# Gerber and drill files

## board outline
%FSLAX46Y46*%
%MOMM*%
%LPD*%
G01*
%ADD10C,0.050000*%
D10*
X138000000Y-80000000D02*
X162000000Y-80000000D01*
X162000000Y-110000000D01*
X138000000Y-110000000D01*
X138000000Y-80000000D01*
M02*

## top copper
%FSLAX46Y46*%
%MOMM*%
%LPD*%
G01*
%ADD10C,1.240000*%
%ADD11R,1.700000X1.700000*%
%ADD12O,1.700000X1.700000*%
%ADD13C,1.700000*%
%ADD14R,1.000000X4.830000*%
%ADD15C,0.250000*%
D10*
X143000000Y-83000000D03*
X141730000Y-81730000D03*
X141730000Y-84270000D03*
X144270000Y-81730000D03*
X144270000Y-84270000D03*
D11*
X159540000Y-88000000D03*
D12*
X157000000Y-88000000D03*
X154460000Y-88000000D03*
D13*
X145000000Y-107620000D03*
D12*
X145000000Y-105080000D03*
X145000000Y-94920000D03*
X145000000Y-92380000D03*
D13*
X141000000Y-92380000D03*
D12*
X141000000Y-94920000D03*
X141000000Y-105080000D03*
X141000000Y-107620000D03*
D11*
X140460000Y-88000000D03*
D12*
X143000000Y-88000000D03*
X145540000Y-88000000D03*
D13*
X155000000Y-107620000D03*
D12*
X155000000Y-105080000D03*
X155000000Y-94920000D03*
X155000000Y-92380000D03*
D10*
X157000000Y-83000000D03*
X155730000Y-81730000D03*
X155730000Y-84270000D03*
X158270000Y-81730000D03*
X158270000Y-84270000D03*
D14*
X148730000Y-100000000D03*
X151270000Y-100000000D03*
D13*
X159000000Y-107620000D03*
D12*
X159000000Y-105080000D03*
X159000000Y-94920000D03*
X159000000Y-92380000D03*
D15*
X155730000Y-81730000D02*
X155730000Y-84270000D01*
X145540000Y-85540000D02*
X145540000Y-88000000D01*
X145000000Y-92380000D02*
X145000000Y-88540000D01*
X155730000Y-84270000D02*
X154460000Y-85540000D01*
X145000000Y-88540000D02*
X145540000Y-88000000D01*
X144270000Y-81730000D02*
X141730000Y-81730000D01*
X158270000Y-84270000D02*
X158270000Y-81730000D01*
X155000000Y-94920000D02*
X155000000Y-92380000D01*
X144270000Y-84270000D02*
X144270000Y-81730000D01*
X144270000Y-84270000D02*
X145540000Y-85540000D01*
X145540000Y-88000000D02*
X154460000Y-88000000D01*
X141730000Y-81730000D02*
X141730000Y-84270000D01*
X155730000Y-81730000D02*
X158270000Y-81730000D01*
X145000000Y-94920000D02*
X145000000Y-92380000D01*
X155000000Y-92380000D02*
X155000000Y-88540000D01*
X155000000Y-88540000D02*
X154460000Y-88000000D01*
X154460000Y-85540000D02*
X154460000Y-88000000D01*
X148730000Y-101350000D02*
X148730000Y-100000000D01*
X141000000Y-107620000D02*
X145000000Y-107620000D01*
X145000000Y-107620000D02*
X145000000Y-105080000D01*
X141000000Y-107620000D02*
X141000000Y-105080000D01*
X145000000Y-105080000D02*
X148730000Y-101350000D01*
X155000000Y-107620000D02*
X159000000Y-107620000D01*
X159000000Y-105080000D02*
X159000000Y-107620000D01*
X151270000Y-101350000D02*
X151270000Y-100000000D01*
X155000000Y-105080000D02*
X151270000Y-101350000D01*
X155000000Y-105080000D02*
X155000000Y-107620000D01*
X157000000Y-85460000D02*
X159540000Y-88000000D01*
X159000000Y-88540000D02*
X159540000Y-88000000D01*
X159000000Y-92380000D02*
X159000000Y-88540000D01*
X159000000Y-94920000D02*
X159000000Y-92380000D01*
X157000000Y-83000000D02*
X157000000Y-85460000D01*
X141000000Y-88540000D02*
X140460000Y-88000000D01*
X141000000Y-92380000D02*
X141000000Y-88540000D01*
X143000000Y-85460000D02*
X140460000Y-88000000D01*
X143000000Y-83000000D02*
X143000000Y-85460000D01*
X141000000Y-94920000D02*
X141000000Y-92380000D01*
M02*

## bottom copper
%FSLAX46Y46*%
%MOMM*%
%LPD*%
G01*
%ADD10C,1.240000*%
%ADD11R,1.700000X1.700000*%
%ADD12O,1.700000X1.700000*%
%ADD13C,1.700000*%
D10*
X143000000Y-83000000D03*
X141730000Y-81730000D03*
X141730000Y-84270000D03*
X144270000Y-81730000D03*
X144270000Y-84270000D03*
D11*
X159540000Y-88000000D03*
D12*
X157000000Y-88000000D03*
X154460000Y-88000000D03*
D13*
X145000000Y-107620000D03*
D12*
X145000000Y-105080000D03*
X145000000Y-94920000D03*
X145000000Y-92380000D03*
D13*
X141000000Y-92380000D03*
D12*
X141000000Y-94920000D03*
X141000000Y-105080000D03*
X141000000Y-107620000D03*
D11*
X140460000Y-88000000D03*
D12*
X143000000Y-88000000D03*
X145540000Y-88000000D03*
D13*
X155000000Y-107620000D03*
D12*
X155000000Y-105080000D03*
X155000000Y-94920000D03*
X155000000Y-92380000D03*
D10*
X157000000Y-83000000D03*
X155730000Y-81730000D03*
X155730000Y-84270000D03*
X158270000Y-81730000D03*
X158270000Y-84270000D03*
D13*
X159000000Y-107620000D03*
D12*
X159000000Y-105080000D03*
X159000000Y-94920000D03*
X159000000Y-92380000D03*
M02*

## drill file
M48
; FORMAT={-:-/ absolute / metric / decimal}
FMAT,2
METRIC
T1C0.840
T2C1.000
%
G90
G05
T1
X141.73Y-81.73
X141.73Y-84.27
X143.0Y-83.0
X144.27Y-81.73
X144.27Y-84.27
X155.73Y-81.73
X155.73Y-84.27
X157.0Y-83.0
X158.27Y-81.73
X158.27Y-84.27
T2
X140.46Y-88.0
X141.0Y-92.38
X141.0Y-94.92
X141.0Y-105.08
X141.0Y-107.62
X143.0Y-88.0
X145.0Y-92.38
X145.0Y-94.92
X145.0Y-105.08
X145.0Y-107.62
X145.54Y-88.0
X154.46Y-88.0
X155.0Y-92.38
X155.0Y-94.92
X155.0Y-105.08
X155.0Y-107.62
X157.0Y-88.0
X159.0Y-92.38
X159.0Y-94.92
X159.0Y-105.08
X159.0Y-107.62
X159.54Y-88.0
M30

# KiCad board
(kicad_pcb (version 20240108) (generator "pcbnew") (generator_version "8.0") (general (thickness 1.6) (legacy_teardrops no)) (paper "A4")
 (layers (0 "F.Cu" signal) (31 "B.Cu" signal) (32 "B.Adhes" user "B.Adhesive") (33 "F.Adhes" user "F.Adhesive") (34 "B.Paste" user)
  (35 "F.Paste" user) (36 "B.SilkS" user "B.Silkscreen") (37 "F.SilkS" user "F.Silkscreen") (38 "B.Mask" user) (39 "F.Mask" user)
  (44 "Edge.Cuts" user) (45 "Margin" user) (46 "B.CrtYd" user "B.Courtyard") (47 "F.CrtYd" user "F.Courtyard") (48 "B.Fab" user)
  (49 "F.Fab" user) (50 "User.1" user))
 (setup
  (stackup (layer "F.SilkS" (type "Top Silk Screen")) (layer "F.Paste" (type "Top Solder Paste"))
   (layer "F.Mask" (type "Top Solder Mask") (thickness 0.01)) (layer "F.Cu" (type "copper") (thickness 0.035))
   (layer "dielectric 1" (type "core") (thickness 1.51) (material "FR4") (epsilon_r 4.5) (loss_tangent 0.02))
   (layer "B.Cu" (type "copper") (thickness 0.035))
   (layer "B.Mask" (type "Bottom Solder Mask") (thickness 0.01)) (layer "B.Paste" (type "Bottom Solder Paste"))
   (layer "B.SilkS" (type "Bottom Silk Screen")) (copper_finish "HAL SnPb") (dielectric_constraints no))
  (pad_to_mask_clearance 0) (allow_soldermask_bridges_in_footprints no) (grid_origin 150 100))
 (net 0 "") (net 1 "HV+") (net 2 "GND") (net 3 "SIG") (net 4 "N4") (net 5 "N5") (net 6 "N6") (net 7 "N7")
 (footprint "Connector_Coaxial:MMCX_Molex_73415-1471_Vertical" (layer "F.Cu") (at 143 83)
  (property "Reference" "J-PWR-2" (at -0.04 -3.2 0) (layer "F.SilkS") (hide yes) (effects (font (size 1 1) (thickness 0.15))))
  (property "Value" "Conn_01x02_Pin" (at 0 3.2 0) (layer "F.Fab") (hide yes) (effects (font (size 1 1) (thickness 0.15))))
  (pad "1" thru_hole circle (at 0 0) (size 1.24 1.24) (drill 0.84) (layers "*.Cu" "*.Mask") (remove_unused_layers no) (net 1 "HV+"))
  (pad "2" thru_hole circle (at -1.27 -1.27) (size 1.24 1.24) (drill 0.84) (layers "*.Cu" "*.Mask") (remove_unused_layers no) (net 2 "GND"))
  (pad "2" thru_hole circle (at -1.27 1.27) (size 1.24 1.24) (drill 0.84) (layers "*.Cu" "*.Mask") (remove_unused_layers no) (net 2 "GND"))
  (pad "2" thru_hole circle (at 1.27 -1.27) (size 1.24 1.24) (drill 0.84) (layers "*.Cu" "*.Mask") (remove_unused_layers no) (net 2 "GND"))
  (pad "2" thru_hole circle (at 1.27 1.27) (size 1.24 1.24) (drill 0.84) (layers "*.Cu" "*.Mask") (remove_unused_layers no) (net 2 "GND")))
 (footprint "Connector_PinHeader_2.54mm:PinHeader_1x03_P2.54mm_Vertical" (layer "F.Cu") (at 159.54 88 -90)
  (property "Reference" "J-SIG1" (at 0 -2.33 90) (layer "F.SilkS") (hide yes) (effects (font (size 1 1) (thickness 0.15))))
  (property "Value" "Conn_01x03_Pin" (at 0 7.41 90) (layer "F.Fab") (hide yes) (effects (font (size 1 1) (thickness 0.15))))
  (pad "1" thru_hole rect (at 0 0 270) (size 1.7 1.7) (drill 1) (layers "*.Cu" "*.Mask") (remove_unused_layers no) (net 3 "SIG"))
  (pad "2" thru_hole oval (at 0 2.54 270) (size 1.7 1.7) (drill 1) (layers "*.Cu" "*.Mask") (remove_unused_layers no) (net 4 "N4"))
  (pad "3" thru_hole oval (at 0 5.08 270) (size 1.7 1.7) (drill 1) (layers "*.Cu" "*.Mask") (remove_unused_layers no) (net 2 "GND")))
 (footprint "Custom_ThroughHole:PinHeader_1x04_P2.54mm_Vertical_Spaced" (layer "F.Cu") (at 145 100 180)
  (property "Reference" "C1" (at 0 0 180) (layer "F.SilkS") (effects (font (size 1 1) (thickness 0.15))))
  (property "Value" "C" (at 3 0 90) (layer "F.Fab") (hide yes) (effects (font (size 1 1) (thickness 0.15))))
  (pad "1" thru_hole circle (at 0 -7.62 180) (size 1.7 1.7) (drill 1) (layers "*.Cu" "*.Mask") (remove_unused_layers no) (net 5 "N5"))
  (pad "1" thru_hole oval (at 0 -5.08 180) (size 1.7 1.7) (drill 1) (layers "*.Cu" "*.Mask") (remove_unused_layers no) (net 5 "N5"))
  (pad "2" thru_hole oval (at 0 5.08 180) (size 1.7 1.7) (drill 1) (layers "*.Cu" "*.Mask") (remove_unused_layers no) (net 2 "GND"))
  (pad "2" thru_hole oval (at 0 7.62 180) (size 1.7 1.7) (drill 1) (layers "*.Cu" "*.Mask") (remove_unused_layers no) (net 2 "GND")))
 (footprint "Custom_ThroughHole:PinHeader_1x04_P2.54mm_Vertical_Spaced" (layer "F.Cu") (at 141 100)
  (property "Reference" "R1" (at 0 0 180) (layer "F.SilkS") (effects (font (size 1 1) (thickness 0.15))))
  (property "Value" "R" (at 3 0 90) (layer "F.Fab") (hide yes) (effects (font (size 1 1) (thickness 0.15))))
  (pad "1" thru_hole circle (at 0 -7.62) (size 1.7 1.7) (drill 1) (layers "*.Cu" "*.Mask") (remove_unused_layers no) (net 1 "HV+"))
  (pad "1" thru_hole oval (at 0 -5.08) (size 1.7 1.7) (drill 1) (layers "*.Cu" "*.Mask") (remove_unused_layers no) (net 1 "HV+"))
  (pad "2" thru_hole oval (at 0 5.08) (size 1.7 1.7) (drill 1) (layers "*.Cu" "*.Mask") (remove_unused_layers no) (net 5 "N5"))
  (pad "2" thru_hole oval (at 0 7.62) (size 1.7 1.7) (drill 1) (layers "*.Cu" "*.Mask") (remove_unused_layers no) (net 5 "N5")))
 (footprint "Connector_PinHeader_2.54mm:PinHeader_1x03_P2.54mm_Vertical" (layer "F.Cu") (at 140.46 88 90)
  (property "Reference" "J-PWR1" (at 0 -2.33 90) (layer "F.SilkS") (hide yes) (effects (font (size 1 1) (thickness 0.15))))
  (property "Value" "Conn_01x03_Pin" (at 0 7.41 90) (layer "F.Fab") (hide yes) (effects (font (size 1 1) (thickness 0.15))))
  (pad "1" thru_hole rect (at 0 0 90) (size 1.7 1.7) (drill 1) (layers "*.Cu" "*.Mask") (remove_unused_layers no) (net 1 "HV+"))
  (pad "2" thru_hole oval (at 0 2.54 90) (size 1.7 1.7) (drill 1) (layers "*.Cu" "*.Mask") (remove_unused_layers no) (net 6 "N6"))
  (pad "3" thru_hole oval (at 0 5.08 90) (size 1.7 1.7) (drill 1) (layers "*.Cu" "*.Mask") (remove_unused_layers no) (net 2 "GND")))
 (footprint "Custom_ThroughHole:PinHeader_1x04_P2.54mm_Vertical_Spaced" (layer "F.Cu") (at 155 100 180)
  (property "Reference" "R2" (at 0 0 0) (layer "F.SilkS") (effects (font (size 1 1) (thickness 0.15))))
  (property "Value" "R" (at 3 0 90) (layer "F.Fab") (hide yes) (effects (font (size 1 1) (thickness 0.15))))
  (pad "1" thru_hole circle (at 0 -7.62 180) (size 1.7 1.7) (drill 1) (layers "*.Cu" "*.Mask") (remove_unused_layers no) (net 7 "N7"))
  (pad "1" thru_hole oval (at 0 -5.08 180) (size 1.7 1.7) (drill 1) (layers "*.Cu" "*.Mask") (remove_unused_layers no) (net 7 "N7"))
  (pad "2" thru_hole oval (at 0 5.08 180) (size 1.7 1.7) (drill 1) (layers "*.Cu" "*.Mask") (remove_unused_layers no) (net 2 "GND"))
  (pad "2" thru_hole oval (at 0 7.62 180) (size 1.7 1.7) (drill 1) (layers "*.Cu" "*.Mask") (remove_unused_layers no) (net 2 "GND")))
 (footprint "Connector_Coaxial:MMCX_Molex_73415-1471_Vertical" (layer "F.Cu") (at 157 83)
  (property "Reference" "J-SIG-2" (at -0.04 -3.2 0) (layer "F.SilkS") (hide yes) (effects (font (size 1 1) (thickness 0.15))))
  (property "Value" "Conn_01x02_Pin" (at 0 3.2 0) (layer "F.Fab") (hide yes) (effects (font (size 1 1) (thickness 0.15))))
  (pad "1" thru_hole circle (at 0 0) (size 1.24 1.24) (drill 0.84) (layers "*.Cu" "*.Mask") (remove_unused_layers no) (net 3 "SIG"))
  (pad "2" thru_hole circle (at -1.27 -1.27) (size 1.24 1.24) (drill 0.84) (layers "*.Cu" "*.Mask") (remove_unused_layers no) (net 2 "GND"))
  (pad "2" thru_hole circle (at -1.27 1.27) (size 1.24 1.24) (drill 0.84) (layers "*.Cu" "*.Mask") (remove_unused_layers no) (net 2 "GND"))
  (pad "2" thru_hole circle (at 1.27 -1.27) (size 1.24 1.24) (drill 0.84) (layers "*.Cu" "*.Mask") (remove_unused_layers no) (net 2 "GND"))
  (pad "2" thru_hole circle (at 1.27 1.27) (size 1.24 1.24) (drill 0.84) (layers "*.Cu" "*.Mask") (remove_unused_layers no) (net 2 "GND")))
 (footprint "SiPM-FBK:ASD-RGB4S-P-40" (layer "F.Cu") (at 150 100)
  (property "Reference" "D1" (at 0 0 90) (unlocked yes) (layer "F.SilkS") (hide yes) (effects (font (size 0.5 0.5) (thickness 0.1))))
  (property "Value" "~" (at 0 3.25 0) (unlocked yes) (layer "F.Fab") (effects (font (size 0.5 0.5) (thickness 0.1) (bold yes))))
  (pad "1" smd rect (at -1.27 0) (size 1 4.83) (layers "F.Cu" "F.Paste" "F.Mask") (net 5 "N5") (thermal_bridge_angle 45))
  (pad "2" smd rect (at 1.27 0) (size 1 4.83) (layers "F.Cu" "F.Paste" "F.Mask") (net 7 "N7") (thermal_bridge_angle 45)))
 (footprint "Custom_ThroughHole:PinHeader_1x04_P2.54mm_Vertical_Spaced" (layer "F.Cu") (at 159 100 180)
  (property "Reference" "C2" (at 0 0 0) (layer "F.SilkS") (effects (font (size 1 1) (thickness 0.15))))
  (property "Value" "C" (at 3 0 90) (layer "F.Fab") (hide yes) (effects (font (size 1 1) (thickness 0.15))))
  (pad "1" thru_hole circle (at 0 -7.62 180) (size 1.7 1.7) (drill 1) (layers "*.Cu" "*.Mask") (remove_unused_layers no) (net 7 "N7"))
  (pad "1" thru_hole oval (at 0 -5.08 180) (size 1.7 1.7) (drill 1) (layers "*.Cu" "*.Mask") (remove_unused_layers no) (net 7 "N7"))
  (pad "2" thru_hole oval (at 0 5.08 180) (size 1.7 1.7) (drill 1) (layers "*.Cu" "*.Mask") (remove_unused_layers no) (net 3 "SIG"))
  (pad "2" thru_hole oval (at 0 7.62 180) (size 1.7 1.7) (drill 1) (layers "*.Cu" "*.Mask") (remove_unused_layers no) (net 3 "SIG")))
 (gr_rect (start 138 80) (end 162 110) (stroke (width 0.05) (type default)) (fill none) (layer "Edge.Cuts"))
 (segment (start 155.73 81.73) (end 155.73 84.27) (width 0.25) (layer "F.Cu") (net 2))
 (segment (start 145.54 85.54) (end 145.54 88) (width 0.25) (layer "F.Cu") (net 2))
 (segment (start 145 92.38) (end 145 88.54) (width 0.25) (layer "F.Cu") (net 2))
 (segment (start 155.73 84.27) (end 154.46 85.54) (width 0.25) (layer "F.Cu") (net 2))
 (segment (start 145 88.54) (end 145.54 88) (width 0.25) (layer "F.Cu") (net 2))
 (segment (start 144.27 81.73) (end 141.73 81.73) (width 0.25) (layer "F.Cu") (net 2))
 (segment (start 158.27 84.27) (end 158.27 81.73) (width 0.25) (layer "F.Cu") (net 2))
 (segment (start 155 94.92) (end 155 92.38) (width 0.25) (layer "F.Cu") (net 2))
 (segment (start 144.27 84.27) (end 144.27 81.73) (width 0.25) (layer "F.Cu") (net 2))
 (segment (start 144.27 84.27) (end 145.54 85.54) (width 0.25) (layer "F.Cu") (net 2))
 (segment (start 145.54 88) (end 154.46 88) (width 0.25) (layer "F.Cu") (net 2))
 (segment (start 141.73 81.73) (end 141.73 84.27) (width 0.25) (layer "F.Cu") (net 2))
 (segment (start 155.73 81.73) (end 158.27 81.73) (width 0.25) (layer "F.Cu") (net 2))
 (segment (start 145 94.92) (end 145 92.38) (width 0.25) (layer "F.Cu") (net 2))
 (segment (start 155 92.38) (end 155 88.54) (width 0.25) (layer "F.Cu") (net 2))
 (segment (start 155 88.54) (end 154.46 88) (width 0.25) (layer "F.Cu") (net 2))
 (segment (start 154.46 85.54) (end 154.46 88) (width 0.25) (layer "F.Cu") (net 2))
 (segment (start 148.73 101.35) (end 148.73 100) (width 0.25) (layer "F.Cu") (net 5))
 (segment (start 141 107.62) (end 145 107.62) (width 0.25) (layer "F.Cu") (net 5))
 (segment (start 145 107.62) (end 145 105.08) (width 0.25) (layer "F.Cu") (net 5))
 (segment (start 141 107.62) (end 141 105.08) (width 0.25) (layer "F.Cu") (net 5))
 (segment (start 145 105.08) (end 148.73 101.35) (width 0.25) (layer "F.Cu") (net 5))
 (segment (start 155 107.62) (end 159 107.62) (width 0.25) (layer "F.Cu") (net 7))
 (segment (start 159 105.08) (end 159 107.62) (width 0.25) (layer "F.Cu") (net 7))
 (segment (start 151.27 101.35) (end 151.27 100) (width 0.25) (layer "F.Cu") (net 7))
 (segment (start 155 105.08) (end 151.27 101.35) (width 0.25) (layer "F.Cu") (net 7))
 (segment (start 155 105.08) (end 155 107.62) (width 0.25) (layer "F.Cu") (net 7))
 (segment (start 157 85.46) (end 159.54 88) (width 0.25) (layer "F.Cu") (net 3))
 (segment (start 159 88.54) (end 159.54 88) (width 0.25) (layer "F.Cu") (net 3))
 (segment (start 159 92.38) (end 159 88.54) (width 0.25) (layer "F.Cu") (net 3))
 (segment (start 159 94.92) (end 159 92.38) (width 0.25) (layer "F.Cu") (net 3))
 (segment (start 157 83) (end 157 85.46) (width 0.25) (layer "F.Cu") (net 3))
 (segment (start 141 88.54) (end 140.46 88) (width 0.25) (layer "F.Cu") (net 1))
 (segment (start 141 92.38) (end 141 88.54) (width 0.25) (layer "F.Cu") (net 1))
 (segment (start 143 85.46) (end 140.46 88) (width 0.25) (layer "F.Cu") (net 1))
 (segment (start 143 83) (end 143 85.46) (width 0.25) (layer "F.Cu") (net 1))
 (segment (start 141 94.92) (end 141 92.38) (width 0.25) (layer "F.Cu") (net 1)))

